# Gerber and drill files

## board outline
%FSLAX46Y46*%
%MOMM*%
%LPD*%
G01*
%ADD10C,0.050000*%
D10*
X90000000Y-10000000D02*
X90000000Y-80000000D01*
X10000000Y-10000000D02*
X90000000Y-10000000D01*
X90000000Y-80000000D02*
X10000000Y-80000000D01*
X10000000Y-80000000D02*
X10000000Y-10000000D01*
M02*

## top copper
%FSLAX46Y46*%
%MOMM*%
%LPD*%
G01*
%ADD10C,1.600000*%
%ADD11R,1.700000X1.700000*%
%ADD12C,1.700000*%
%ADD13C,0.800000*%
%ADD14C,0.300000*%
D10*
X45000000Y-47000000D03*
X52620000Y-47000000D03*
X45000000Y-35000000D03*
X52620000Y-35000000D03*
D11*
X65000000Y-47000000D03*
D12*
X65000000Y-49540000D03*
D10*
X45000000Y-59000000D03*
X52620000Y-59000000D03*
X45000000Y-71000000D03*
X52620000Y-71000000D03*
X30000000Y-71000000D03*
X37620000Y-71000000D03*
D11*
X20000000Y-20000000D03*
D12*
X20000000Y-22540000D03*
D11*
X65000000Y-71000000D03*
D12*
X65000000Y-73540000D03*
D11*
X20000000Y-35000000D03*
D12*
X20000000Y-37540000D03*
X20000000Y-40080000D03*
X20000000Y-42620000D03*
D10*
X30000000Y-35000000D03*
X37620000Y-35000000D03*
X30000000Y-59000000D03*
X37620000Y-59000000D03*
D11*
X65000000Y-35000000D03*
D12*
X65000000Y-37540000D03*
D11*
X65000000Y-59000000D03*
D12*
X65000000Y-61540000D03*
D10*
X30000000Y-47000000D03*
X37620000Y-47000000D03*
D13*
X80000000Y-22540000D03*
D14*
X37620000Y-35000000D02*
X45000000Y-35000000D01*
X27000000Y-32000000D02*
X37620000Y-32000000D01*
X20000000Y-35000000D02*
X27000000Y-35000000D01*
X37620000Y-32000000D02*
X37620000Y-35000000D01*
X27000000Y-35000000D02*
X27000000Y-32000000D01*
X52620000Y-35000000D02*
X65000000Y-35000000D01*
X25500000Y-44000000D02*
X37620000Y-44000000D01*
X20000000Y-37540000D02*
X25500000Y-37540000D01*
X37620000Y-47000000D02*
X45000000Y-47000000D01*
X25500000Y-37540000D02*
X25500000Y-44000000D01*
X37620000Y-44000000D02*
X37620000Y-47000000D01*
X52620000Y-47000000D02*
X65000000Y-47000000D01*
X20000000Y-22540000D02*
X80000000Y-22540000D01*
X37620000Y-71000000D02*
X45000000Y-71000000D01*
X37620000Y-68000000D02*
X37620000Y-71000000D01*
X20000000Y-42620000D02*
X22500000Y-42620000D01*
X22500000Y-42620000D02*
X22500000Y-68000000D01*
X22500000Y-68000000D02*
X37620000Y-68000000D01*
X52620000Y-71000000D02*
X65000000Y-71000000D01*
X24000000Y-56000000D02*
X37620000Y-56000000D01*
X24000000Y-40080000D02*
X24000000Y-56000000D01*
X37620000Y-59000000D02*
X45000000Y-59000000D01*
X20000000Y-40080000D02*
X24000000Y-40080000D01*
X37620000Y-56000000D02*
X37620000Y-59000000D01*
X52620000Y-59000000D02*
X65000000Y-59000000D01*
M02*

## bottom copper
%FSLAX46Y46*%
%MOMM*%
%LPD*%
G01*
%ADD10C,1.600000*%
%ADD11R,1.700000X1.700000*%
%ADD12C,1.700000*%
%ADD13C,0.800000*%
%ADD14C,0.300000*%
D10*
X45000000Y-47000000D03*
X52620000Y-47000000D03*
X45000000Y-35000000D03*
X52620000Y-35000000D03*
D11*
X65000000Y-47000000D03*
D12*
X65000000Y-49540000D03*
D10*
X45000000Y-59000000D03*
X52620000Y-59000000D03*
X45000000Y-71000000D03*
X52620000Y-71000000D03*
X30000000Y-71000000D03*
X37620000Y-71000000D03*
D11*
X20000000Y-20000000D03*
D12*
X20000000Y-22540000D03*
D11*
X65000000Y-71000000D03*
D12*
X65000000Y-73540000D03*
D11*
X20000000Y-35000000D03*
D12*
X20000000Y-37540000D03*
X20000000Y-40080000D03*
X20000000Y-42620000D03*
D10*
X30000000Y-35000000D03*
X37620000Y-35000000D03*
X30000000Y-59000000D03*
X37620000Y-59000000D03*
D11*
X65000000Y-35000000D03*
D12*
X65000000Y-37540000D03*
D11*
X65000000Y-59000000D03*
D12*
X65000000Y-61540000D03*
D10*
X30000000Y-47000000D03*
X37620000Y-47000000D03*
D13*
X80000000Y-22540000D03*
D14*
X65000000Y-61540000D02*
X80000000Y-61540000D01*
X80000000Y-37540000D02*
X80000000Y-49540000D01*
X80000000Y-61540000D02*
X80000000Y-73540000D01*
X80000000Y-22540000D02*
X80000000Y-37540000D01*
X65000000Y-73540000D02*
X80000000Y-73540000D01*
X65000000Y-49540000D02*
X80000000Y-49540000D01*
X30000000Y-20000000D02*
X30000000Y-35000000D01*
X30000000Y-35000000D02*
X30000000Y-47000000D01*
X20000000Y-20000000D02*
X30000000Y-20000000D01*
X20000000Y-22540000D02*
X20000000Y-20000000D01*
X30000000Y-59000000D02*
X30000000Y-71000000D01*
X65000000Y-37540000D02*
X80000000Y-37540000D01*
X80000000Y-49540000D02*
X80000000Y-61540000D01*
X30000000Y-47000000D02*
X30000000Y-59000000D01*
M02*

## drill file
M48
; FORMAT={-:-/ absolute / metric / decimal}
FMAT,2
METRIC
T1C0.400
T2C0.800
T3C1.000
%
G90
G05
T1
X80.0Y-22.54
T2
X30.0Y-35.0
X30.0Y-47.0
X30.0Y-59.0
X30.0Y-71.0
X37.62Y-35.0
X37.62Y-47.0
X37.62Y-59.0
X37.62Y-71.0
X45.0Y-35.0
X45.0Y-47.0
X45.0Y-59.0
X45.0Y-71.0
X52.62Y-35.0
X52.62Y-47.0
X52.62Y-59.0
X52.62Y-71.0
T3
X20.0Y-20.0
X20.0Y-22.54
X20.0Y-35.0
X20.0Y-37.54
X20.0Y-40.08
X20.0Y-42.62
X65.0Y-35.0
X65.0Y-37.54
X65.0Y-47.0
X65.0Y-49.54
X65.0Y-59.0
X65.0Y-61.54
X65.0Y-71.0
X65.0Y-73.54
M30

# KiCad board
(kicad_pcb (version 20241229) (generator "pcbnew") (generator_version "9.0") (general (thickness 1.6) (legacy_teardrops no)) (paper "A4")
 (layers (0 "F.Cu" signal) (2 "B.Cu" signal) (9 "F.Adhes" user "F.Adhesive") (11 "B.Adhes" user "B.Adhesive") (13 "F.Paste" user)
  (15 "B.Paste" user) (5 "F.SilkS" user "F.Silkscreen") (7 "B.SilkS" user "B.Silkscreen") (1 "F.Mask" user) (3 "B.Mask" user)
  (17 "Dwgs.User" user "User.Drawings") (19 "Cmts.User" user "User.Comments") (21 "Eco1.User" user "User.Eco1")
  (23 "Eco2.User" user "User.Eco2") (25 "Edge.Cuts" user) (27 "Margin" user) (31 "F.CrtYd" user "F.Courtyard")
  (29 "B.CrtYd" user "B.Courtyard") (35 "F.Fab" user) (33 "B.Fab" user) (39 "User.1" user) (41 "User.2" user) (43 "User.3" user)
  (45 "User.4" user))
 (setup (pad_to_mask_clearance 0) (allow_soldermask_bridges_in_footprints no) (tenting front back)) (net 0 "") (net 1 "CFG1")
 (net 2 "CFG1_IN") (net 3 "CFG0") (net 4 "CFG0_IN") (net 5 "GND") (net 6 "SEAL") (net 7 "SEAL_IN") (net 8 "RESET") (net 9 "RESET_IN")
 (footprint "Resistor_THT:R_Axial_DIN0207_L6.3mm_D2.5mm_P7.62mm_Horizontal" (layer "F.Cu") (at 45 47)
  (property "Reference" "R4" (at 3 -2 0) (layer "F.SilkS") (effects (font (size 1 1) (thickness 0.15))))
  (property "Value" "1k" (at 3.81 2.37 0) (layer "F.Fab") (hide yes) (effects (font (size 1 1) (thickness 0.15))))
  (pad "1" thru_hole circle (at 0 0) (size 1.6 1.6) (drill 0.8) (layers "*.Cu" "*.Mask") (remove_unused_layers no) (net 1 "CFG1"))
  (pad "2" thru_hole circle (at 7.62 0) (size 1.6 1.6) (drill 0.8) (layers "*.Cu" "*.Mask") (remove_unused_layers no) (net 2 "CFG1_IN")))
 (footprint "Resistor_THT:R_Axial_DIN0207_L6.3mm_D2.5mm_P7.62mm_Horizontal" (layer "F.Cu") (at 45 35)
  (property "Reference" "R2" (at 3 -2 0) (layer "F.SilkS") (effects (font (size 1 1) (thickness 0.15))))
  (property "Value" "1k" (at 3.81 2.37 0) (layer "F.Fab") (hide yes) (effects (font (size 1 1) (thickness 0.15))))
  (pad "1" thru_hole circle (at 0 0) (size 1.6 1.6) (drill 0.8) (layers "*.Cu" "*.Mask") (remove_unused_layers no) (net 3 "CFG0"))
  (pad "2" thru_hole circle (at 7.62 0) (size 1.6 1.6) (drill 0.8) (layers "*.Cu" "*.Mask") (remove_unused_layers no) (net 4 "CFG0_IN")))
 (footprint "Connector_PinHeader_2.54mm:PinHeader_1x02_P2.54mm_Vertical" (layer "F.Cu") (at 65 47)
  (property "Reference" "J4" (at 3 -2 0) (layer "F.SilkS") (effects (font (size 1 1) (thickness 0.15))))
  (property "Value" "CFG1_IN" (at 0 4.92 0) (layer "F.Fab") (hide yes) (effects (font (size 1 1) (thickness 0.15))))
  (pad "1" thru_hole rect (at 0 0) (size 1.7 1.7) (drill 1) (layers "*.Cu" "*.Mask") (remove_unused_layers no) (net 2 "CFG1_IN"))
  (pad "2" thru_hole circle (at 0 2.54) (size 1.7 1.7) (drill 1) (layers "*.Cu" "*.Mask") (remove_unused_layers no) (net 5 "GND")))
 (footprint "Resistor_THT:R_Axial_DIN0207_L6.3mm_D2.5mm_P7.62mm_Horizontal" (layer "F.Cu") (at 45 59)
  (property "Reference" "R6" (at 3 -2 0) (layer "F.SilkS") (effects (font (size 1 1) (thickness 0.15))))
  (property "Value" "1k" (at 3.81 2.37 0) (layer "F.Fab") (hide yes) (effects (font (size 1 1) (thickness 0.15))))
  (pad "1" thru_hole circle (at 0 0) (size 1.6 1.6) (drill 0.8) (layers "*.Cu" "*.Mask") (remove_unused_layers no) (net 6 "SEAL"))
  (pad "2" thru_hole circle (at 7.62 0) (size 1.6 1.6) (drill 0.8) (layers "*.Cu" "*.Mask") (remove_unused_layers no) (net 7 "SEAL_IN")))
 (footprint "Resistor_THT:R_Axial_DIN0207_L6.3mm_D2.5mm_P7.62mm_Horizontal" (layer "F.Cu") (at 45 71)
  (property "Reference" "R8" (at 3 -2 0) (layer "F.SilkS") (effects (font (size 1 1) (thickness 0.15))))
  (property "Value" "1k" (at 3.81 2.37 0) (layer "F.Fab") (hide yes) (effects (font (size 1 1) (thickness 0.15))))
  (pad "1" thru_hole circle (at 0 0) (size 1.6 1.6) (drill 0.8) (layers "*.Cu" "*.Mask") (remove_unused_layers no) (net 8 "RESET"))
  (pad "2" thru_hole circle (at 7.62 0) (size 1.6 1.6) (drill 0.8) (layers "*.Cu" "*.Mask") (remove_unused_layers no) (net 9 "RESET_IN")))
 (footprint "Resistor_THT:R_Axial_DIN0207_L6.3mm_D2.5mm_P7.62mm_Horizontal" (layer "F.Cu") (at 30 71)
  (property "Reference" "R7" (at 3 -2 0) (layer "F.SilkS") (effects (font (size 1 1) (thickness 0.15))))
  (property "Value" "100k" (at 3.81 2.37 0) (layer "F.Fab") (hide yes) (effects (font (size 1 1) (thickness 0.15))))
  (pad "1" thru_hole circle (at 0 0) (size 1.6 1.6) (drill 0.8) (layers "*.Cu" "*.Mask") (remove_unused_layers no) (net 5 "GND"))
  (pad "2" thru_hole circle (at 7.62 0) (size 1.6 1.6) (drill 0.8) (layers "*.Cu" "*.Mask") (remove_unused_layers no) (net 8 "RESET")))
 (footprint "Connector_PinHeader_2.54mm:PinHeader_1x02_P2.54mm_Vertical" (layer "F.Cu") (at 20 20)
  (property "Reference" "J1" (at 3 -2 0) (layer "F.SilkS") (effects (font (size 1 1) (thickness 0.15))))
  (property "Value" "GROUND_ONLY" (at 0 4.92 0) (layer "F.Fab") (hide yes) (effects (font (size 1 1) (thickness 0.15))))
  (pad "1" thru_hole rect (at 0 0) (size 1.7 1.7) (drill 1) (layers "*.Cu" "*.Mask") (remove_unused_layers no) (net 5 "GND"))
  (pad "2" thru_hole circle (at 0 2.54) (size 1.7 1.7) (drill 1) (layers "*.Cu" "*.Mask") (remove_unused_layers no) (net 5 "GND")))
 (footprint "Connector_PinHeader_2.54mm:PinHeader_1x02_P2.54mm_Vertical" (layer "F.Cu") (at 65 71)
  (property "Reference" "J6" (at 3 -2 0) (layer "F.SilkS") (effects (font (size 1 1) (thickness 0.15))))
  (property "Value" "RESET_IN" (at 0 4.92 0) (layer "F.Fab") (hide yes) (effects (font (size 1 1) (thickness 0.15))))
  (pad "1" thru_hole rect (at 0 0) (size 1.7 1.7) (drill 1) (layers "*.Cu" "*.Mask") (remove_unused_layers no) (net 9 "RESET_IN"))
  (pad "2" thru_hole circle (at 0 2.54) (size 1.7 1.7) (drill 1) (layers "*.Cu" "*.Mask") (remove_unused_layers no) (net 5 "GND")))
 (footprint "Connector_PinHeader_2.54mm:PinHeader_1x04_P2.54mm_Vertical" (layer "F.Cu") (at 20 35)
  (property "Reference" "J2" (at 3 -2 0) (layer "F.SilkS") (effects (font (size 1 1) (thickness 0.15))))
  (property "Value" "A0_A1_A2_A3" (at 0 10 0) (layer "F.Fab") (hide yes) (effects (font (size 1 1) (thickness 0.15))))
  (pad "1" thru_hole rect (at 0 0) (size 1.7 1.7) (drill 1) (layers "*.Cu" "*.Mask") (remove_unused_layers no) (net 3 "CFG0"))
  (pad "2" thru_hole circle (at 0 2.54) (size 1.7 1.7) (drill 1) (layers "*.Cu" "*.Mask") (remove_unused_layers no) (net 1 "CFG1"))
  (pad "3" thru_hole circle (at 0 5.08) (size 1.7 1.7) (drill 1) (layers "*.Cu" "*.Mask") (remove_unused_layers no) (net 6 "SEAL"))
  (pad "4" thru_hole circle (at 0 7.62) (size 1.7 1.7) (drill 1) (layers "*.Cu" "*.Mask") (remove_unused_layers no) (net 8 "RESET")))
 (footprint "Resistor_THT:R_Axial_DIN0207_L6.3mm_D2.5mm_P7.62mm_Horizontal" (layer "F.Cu") (at 30 35)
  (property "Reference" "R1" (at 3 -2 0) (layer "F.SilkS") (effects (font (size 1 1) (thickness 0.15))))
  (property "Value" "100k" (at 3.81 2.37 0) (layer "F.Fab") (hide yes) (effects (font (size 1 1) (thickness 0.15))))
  (pad "1" thru_hole circle (at 0 0) (size 1.6 1.6) (drill 0.8) (layers "*.Cu" "*.Mask") (remove_unused_layers no) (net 5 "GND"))
  (pad "2" thru_hole circle (at 7.62 0) (size 1.6 1.6) (drill 0.8) (layers "*.Cu" "*.Mask") (remove_unused_layers no) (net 3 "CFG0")))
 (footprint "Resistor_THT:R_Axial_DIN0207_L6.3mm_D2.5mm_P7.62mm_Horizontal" (layer "F.Cu") (at 30 59)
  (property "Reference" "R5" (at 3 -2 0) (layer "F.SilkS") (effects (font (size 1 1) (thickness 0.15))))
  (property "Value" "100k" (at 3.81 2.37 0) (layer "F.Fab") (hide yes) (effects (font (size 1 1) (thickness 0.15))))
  (pad "1" thru_hole circle (at 0 0) (size 1.6 1.6) (drill 0.8) (layers "*.Cu" "*.Mask") (remove_unused_layers no) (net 5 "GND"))
  (pad "2" thru_hole circle (at 7.62 0) (size 1.6 1.6) (drill 0.8) (layers "*.Cu" "*.Mask") (remove_unused_layers no) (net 6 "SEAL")))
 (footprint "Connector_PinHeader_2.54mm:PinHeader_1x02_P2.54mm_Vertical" (layer "F.Cu") (at 65 35)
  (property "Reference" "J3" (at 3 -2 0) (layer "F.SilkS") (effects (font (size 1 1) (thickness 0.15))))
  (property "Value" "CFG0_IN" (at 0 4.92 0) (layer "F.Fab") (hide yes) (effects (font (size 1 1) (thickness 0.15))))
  (pad "1" thru_hole rect (at 0 0) (size 1.7 1.7) (drill 1) (layers "*.Cu" "*.Mask") (remove_unused_layers no) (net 4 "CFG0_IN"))
  (pad "2" thru_hole circle (at 0 2.54) (size 1.7 1.7) (drill 1) (layers "*.Cu" "*.Mask") (remove_unused_layers no) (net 5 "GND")))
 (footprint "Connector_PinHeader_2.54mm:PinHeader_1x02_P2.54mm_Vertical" (layer "F.Cu") (at 65 59)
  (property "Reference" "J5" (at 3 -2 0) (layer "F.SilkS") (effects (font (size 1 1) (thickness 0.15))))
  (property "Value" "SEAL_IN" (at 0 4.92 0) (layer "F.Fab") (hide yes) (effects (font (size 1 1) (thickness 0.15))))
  (pad "1" thru_hole rect (at 0 0) (size 1.7 1.7) (drill 1) (layers "*.Cu" "*.Mask") (remove_unused_layers no) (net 7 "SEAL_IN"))
  (pad "2" thru_hole circle (at 0 2.54) (size 1.7 1.7) (drill 1) (layers "*.Cu" "*.Mask") (remove_unused_layers no) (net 5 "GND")))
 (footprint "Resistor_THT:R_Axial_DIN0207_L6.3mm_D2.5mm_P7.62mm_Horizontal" (layer "F.Cu") (at 30 47)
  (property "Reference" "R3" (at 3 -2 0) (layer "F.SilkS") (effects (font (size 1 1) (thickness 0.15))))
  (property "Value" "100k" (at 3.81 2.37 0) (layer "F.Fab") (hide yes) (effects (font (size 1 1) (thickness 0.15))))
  (pad "1" thru_hole circle (at 0 0) (size 1.6 1.6) (drill 0.8) (layers "*.Cu" "*.Mask") (remove_unused_layers no) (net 5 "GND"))
  (pad "2" thru_hole circle (at 7.62 0) (size 1.6 1.6) (drill 0.8) (layers "*.Cu" "*.Mask") (remove_unused_layers no) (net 1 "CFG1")))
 (gr_line (start 90 10) (end 90 80) (stroke (width 0.05) (type default)) (layer "Edge.Cuts"))
 (gr_line (start 10 10) (end 90 10) (stroke (width 0.05) (type default)) (layer "Edge.Cuts"))
 (gr_line (start 90 80) (end 10 80) (stroke (width 0.05) (type default)) (layer "Edge.Cuts"))
 (gr_line (start 10 80) (end 10 10) (stroke (width 0.05) (type default)) (layer "Edge.Cuts"))
 (segment (start 37.62 35) (end 45 35) (width 0.3) (layer "F.Cu") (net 3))
 (segment (start 27 32) (end 37.62 32) (width 0.3) (layer "F.Cu") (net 3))
 (segment (start 20 35) (end 27 35) (width 0.3) (layer "F.Cu") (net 3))
 (segment (start 37.62 32) (end 37.62 35) (width 0.3) (layer "F.Cu") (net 3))
 (segment (start 27 35) (end 27 32) (width 0.3) (layer "F.Cu") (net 3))
 (segment (start 52.62 35) (end 65 35) (width 0.3) (layer "F.Cu") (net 4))
 (segment (start 25.5 44) (end 37.62 44) (width 0.3) (layer "F.Cu") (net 1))
 (segment (start 20 37.54) (end 25.5 37.54) (width 0.3) (layer "F.Cu") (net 1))
 (segment (start 37.62 47) (end 45 47) (width 0.3) (layer "F.Cu") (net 1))
 (segment (start 25.5 37.54) (end 25.5 44) (width 0.3) (layer "F.Cu") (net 1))
 (segment (start 37.62 44) (end 37.62 47) (width 0.3) (layer "F.Cu") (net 1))
 (segment (start 52.62 47) (end 65 47) (width 0.3) (layer "F.Cu") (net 2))
 (segment (start 20 22.54) (end 80 22.54) (width 0.3) (layer "F.Cu") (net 5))
 (via (at 80 22.54) (size 0.8) (drill 0.4) (layers "F.Cu" "B.Cu") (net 5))
 (segment (start 65 61.54) (end 80 61.54) (width 0.3) (layer "B.Cu") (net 5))
 (segment (start 80 37.54) (end 80 49.54) (width 0.3) (layer "B.Cu") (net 5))
 (segment (start 80 61.54) (end 80 73.54) (width 0.3) (layer "B.Cu") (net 5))
 (segment (start 80 22.54) (end 80 37.54) (width 0.3) (layer "B.Cu") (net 5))
 (segment (start 65 73.54) (end 80 73.54) (width 0.3) (layer "B.Cu") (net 5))
 (segment (start 65 49.54) (end 80 49.54) (width 0.3) (layer "B.Cu") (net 5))
 (segment (start 30 20) (end 30 35) (width 0.3) (layer "B.Cu") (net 5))
 (segment (start 30 35) (end 30 47) (width 0.3) (layer "B.Cu") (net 5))
 (segment (start 20 20) (end 30 20) (width 0.3) (layer "B.Cu") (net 5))
 (segment (start 20 22.54) (end 20 20) (width 0.3) (layer "B.Cu") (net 5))
 (segment (start 30 59) (end 30 71) (width 0.3) (layer "B.Cu") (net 5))
 (segment (start 65 37.54) (end 80 37.54) (width 0.3) (layer "B.Cu") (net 5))
 (segment (start 80 49.54) (end 80 61.54) (width 0.3) (layer "B.Cu") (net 5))
 (segment (start 30 47) (end 30 59) (width 0.3) (layer "B.Cu") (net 5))
 (segment (start 37.62 71) (end 45 71) (width 0.3) (layer "F.Cu") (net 8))
 (segment (start 37.62 68) (end 37.62 71) (width 0.3) (layer "F.Cu") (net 8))
 (segment (start 20 42.62) (end 22.5 42.62) (width 0.3) (layer "F.Cu") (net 8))
 (segment (start 22.5 42.62) (end 22.5 68) (width 0.3) (layer "F.Cu") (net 8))
 (segment (start 22.5 68) (end 37.62 68) (width 0.3) (layer "F.Cu") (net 8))
 (segment (start 52.62 71) (end 65 71) (width 0.3) (layer "F.Cu") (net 9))
 (segment (start 24 56) (end 37.62 56) (width 0.3) (layer "F.Cu") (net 6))
 (segment (start 24 40.08) (end 24 56) (width 0.3) (layer "F.Cu") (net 6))
 (segment (start 37.62 59) (end 45 59) (width 0.3) (layer "F.Cu") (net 6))
 (segment (start 20 40.08) (end 24 40.08) (width 0.3) (layer "F.Cu") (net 6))
 (segment (start 37.62 56) (end 37.62 59) (width 0.3) (layer "F.Cu") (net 6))
 (segment (start 52.62 59) (end 65 59) (width 0.3) (layer "F.Cu") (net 7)))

